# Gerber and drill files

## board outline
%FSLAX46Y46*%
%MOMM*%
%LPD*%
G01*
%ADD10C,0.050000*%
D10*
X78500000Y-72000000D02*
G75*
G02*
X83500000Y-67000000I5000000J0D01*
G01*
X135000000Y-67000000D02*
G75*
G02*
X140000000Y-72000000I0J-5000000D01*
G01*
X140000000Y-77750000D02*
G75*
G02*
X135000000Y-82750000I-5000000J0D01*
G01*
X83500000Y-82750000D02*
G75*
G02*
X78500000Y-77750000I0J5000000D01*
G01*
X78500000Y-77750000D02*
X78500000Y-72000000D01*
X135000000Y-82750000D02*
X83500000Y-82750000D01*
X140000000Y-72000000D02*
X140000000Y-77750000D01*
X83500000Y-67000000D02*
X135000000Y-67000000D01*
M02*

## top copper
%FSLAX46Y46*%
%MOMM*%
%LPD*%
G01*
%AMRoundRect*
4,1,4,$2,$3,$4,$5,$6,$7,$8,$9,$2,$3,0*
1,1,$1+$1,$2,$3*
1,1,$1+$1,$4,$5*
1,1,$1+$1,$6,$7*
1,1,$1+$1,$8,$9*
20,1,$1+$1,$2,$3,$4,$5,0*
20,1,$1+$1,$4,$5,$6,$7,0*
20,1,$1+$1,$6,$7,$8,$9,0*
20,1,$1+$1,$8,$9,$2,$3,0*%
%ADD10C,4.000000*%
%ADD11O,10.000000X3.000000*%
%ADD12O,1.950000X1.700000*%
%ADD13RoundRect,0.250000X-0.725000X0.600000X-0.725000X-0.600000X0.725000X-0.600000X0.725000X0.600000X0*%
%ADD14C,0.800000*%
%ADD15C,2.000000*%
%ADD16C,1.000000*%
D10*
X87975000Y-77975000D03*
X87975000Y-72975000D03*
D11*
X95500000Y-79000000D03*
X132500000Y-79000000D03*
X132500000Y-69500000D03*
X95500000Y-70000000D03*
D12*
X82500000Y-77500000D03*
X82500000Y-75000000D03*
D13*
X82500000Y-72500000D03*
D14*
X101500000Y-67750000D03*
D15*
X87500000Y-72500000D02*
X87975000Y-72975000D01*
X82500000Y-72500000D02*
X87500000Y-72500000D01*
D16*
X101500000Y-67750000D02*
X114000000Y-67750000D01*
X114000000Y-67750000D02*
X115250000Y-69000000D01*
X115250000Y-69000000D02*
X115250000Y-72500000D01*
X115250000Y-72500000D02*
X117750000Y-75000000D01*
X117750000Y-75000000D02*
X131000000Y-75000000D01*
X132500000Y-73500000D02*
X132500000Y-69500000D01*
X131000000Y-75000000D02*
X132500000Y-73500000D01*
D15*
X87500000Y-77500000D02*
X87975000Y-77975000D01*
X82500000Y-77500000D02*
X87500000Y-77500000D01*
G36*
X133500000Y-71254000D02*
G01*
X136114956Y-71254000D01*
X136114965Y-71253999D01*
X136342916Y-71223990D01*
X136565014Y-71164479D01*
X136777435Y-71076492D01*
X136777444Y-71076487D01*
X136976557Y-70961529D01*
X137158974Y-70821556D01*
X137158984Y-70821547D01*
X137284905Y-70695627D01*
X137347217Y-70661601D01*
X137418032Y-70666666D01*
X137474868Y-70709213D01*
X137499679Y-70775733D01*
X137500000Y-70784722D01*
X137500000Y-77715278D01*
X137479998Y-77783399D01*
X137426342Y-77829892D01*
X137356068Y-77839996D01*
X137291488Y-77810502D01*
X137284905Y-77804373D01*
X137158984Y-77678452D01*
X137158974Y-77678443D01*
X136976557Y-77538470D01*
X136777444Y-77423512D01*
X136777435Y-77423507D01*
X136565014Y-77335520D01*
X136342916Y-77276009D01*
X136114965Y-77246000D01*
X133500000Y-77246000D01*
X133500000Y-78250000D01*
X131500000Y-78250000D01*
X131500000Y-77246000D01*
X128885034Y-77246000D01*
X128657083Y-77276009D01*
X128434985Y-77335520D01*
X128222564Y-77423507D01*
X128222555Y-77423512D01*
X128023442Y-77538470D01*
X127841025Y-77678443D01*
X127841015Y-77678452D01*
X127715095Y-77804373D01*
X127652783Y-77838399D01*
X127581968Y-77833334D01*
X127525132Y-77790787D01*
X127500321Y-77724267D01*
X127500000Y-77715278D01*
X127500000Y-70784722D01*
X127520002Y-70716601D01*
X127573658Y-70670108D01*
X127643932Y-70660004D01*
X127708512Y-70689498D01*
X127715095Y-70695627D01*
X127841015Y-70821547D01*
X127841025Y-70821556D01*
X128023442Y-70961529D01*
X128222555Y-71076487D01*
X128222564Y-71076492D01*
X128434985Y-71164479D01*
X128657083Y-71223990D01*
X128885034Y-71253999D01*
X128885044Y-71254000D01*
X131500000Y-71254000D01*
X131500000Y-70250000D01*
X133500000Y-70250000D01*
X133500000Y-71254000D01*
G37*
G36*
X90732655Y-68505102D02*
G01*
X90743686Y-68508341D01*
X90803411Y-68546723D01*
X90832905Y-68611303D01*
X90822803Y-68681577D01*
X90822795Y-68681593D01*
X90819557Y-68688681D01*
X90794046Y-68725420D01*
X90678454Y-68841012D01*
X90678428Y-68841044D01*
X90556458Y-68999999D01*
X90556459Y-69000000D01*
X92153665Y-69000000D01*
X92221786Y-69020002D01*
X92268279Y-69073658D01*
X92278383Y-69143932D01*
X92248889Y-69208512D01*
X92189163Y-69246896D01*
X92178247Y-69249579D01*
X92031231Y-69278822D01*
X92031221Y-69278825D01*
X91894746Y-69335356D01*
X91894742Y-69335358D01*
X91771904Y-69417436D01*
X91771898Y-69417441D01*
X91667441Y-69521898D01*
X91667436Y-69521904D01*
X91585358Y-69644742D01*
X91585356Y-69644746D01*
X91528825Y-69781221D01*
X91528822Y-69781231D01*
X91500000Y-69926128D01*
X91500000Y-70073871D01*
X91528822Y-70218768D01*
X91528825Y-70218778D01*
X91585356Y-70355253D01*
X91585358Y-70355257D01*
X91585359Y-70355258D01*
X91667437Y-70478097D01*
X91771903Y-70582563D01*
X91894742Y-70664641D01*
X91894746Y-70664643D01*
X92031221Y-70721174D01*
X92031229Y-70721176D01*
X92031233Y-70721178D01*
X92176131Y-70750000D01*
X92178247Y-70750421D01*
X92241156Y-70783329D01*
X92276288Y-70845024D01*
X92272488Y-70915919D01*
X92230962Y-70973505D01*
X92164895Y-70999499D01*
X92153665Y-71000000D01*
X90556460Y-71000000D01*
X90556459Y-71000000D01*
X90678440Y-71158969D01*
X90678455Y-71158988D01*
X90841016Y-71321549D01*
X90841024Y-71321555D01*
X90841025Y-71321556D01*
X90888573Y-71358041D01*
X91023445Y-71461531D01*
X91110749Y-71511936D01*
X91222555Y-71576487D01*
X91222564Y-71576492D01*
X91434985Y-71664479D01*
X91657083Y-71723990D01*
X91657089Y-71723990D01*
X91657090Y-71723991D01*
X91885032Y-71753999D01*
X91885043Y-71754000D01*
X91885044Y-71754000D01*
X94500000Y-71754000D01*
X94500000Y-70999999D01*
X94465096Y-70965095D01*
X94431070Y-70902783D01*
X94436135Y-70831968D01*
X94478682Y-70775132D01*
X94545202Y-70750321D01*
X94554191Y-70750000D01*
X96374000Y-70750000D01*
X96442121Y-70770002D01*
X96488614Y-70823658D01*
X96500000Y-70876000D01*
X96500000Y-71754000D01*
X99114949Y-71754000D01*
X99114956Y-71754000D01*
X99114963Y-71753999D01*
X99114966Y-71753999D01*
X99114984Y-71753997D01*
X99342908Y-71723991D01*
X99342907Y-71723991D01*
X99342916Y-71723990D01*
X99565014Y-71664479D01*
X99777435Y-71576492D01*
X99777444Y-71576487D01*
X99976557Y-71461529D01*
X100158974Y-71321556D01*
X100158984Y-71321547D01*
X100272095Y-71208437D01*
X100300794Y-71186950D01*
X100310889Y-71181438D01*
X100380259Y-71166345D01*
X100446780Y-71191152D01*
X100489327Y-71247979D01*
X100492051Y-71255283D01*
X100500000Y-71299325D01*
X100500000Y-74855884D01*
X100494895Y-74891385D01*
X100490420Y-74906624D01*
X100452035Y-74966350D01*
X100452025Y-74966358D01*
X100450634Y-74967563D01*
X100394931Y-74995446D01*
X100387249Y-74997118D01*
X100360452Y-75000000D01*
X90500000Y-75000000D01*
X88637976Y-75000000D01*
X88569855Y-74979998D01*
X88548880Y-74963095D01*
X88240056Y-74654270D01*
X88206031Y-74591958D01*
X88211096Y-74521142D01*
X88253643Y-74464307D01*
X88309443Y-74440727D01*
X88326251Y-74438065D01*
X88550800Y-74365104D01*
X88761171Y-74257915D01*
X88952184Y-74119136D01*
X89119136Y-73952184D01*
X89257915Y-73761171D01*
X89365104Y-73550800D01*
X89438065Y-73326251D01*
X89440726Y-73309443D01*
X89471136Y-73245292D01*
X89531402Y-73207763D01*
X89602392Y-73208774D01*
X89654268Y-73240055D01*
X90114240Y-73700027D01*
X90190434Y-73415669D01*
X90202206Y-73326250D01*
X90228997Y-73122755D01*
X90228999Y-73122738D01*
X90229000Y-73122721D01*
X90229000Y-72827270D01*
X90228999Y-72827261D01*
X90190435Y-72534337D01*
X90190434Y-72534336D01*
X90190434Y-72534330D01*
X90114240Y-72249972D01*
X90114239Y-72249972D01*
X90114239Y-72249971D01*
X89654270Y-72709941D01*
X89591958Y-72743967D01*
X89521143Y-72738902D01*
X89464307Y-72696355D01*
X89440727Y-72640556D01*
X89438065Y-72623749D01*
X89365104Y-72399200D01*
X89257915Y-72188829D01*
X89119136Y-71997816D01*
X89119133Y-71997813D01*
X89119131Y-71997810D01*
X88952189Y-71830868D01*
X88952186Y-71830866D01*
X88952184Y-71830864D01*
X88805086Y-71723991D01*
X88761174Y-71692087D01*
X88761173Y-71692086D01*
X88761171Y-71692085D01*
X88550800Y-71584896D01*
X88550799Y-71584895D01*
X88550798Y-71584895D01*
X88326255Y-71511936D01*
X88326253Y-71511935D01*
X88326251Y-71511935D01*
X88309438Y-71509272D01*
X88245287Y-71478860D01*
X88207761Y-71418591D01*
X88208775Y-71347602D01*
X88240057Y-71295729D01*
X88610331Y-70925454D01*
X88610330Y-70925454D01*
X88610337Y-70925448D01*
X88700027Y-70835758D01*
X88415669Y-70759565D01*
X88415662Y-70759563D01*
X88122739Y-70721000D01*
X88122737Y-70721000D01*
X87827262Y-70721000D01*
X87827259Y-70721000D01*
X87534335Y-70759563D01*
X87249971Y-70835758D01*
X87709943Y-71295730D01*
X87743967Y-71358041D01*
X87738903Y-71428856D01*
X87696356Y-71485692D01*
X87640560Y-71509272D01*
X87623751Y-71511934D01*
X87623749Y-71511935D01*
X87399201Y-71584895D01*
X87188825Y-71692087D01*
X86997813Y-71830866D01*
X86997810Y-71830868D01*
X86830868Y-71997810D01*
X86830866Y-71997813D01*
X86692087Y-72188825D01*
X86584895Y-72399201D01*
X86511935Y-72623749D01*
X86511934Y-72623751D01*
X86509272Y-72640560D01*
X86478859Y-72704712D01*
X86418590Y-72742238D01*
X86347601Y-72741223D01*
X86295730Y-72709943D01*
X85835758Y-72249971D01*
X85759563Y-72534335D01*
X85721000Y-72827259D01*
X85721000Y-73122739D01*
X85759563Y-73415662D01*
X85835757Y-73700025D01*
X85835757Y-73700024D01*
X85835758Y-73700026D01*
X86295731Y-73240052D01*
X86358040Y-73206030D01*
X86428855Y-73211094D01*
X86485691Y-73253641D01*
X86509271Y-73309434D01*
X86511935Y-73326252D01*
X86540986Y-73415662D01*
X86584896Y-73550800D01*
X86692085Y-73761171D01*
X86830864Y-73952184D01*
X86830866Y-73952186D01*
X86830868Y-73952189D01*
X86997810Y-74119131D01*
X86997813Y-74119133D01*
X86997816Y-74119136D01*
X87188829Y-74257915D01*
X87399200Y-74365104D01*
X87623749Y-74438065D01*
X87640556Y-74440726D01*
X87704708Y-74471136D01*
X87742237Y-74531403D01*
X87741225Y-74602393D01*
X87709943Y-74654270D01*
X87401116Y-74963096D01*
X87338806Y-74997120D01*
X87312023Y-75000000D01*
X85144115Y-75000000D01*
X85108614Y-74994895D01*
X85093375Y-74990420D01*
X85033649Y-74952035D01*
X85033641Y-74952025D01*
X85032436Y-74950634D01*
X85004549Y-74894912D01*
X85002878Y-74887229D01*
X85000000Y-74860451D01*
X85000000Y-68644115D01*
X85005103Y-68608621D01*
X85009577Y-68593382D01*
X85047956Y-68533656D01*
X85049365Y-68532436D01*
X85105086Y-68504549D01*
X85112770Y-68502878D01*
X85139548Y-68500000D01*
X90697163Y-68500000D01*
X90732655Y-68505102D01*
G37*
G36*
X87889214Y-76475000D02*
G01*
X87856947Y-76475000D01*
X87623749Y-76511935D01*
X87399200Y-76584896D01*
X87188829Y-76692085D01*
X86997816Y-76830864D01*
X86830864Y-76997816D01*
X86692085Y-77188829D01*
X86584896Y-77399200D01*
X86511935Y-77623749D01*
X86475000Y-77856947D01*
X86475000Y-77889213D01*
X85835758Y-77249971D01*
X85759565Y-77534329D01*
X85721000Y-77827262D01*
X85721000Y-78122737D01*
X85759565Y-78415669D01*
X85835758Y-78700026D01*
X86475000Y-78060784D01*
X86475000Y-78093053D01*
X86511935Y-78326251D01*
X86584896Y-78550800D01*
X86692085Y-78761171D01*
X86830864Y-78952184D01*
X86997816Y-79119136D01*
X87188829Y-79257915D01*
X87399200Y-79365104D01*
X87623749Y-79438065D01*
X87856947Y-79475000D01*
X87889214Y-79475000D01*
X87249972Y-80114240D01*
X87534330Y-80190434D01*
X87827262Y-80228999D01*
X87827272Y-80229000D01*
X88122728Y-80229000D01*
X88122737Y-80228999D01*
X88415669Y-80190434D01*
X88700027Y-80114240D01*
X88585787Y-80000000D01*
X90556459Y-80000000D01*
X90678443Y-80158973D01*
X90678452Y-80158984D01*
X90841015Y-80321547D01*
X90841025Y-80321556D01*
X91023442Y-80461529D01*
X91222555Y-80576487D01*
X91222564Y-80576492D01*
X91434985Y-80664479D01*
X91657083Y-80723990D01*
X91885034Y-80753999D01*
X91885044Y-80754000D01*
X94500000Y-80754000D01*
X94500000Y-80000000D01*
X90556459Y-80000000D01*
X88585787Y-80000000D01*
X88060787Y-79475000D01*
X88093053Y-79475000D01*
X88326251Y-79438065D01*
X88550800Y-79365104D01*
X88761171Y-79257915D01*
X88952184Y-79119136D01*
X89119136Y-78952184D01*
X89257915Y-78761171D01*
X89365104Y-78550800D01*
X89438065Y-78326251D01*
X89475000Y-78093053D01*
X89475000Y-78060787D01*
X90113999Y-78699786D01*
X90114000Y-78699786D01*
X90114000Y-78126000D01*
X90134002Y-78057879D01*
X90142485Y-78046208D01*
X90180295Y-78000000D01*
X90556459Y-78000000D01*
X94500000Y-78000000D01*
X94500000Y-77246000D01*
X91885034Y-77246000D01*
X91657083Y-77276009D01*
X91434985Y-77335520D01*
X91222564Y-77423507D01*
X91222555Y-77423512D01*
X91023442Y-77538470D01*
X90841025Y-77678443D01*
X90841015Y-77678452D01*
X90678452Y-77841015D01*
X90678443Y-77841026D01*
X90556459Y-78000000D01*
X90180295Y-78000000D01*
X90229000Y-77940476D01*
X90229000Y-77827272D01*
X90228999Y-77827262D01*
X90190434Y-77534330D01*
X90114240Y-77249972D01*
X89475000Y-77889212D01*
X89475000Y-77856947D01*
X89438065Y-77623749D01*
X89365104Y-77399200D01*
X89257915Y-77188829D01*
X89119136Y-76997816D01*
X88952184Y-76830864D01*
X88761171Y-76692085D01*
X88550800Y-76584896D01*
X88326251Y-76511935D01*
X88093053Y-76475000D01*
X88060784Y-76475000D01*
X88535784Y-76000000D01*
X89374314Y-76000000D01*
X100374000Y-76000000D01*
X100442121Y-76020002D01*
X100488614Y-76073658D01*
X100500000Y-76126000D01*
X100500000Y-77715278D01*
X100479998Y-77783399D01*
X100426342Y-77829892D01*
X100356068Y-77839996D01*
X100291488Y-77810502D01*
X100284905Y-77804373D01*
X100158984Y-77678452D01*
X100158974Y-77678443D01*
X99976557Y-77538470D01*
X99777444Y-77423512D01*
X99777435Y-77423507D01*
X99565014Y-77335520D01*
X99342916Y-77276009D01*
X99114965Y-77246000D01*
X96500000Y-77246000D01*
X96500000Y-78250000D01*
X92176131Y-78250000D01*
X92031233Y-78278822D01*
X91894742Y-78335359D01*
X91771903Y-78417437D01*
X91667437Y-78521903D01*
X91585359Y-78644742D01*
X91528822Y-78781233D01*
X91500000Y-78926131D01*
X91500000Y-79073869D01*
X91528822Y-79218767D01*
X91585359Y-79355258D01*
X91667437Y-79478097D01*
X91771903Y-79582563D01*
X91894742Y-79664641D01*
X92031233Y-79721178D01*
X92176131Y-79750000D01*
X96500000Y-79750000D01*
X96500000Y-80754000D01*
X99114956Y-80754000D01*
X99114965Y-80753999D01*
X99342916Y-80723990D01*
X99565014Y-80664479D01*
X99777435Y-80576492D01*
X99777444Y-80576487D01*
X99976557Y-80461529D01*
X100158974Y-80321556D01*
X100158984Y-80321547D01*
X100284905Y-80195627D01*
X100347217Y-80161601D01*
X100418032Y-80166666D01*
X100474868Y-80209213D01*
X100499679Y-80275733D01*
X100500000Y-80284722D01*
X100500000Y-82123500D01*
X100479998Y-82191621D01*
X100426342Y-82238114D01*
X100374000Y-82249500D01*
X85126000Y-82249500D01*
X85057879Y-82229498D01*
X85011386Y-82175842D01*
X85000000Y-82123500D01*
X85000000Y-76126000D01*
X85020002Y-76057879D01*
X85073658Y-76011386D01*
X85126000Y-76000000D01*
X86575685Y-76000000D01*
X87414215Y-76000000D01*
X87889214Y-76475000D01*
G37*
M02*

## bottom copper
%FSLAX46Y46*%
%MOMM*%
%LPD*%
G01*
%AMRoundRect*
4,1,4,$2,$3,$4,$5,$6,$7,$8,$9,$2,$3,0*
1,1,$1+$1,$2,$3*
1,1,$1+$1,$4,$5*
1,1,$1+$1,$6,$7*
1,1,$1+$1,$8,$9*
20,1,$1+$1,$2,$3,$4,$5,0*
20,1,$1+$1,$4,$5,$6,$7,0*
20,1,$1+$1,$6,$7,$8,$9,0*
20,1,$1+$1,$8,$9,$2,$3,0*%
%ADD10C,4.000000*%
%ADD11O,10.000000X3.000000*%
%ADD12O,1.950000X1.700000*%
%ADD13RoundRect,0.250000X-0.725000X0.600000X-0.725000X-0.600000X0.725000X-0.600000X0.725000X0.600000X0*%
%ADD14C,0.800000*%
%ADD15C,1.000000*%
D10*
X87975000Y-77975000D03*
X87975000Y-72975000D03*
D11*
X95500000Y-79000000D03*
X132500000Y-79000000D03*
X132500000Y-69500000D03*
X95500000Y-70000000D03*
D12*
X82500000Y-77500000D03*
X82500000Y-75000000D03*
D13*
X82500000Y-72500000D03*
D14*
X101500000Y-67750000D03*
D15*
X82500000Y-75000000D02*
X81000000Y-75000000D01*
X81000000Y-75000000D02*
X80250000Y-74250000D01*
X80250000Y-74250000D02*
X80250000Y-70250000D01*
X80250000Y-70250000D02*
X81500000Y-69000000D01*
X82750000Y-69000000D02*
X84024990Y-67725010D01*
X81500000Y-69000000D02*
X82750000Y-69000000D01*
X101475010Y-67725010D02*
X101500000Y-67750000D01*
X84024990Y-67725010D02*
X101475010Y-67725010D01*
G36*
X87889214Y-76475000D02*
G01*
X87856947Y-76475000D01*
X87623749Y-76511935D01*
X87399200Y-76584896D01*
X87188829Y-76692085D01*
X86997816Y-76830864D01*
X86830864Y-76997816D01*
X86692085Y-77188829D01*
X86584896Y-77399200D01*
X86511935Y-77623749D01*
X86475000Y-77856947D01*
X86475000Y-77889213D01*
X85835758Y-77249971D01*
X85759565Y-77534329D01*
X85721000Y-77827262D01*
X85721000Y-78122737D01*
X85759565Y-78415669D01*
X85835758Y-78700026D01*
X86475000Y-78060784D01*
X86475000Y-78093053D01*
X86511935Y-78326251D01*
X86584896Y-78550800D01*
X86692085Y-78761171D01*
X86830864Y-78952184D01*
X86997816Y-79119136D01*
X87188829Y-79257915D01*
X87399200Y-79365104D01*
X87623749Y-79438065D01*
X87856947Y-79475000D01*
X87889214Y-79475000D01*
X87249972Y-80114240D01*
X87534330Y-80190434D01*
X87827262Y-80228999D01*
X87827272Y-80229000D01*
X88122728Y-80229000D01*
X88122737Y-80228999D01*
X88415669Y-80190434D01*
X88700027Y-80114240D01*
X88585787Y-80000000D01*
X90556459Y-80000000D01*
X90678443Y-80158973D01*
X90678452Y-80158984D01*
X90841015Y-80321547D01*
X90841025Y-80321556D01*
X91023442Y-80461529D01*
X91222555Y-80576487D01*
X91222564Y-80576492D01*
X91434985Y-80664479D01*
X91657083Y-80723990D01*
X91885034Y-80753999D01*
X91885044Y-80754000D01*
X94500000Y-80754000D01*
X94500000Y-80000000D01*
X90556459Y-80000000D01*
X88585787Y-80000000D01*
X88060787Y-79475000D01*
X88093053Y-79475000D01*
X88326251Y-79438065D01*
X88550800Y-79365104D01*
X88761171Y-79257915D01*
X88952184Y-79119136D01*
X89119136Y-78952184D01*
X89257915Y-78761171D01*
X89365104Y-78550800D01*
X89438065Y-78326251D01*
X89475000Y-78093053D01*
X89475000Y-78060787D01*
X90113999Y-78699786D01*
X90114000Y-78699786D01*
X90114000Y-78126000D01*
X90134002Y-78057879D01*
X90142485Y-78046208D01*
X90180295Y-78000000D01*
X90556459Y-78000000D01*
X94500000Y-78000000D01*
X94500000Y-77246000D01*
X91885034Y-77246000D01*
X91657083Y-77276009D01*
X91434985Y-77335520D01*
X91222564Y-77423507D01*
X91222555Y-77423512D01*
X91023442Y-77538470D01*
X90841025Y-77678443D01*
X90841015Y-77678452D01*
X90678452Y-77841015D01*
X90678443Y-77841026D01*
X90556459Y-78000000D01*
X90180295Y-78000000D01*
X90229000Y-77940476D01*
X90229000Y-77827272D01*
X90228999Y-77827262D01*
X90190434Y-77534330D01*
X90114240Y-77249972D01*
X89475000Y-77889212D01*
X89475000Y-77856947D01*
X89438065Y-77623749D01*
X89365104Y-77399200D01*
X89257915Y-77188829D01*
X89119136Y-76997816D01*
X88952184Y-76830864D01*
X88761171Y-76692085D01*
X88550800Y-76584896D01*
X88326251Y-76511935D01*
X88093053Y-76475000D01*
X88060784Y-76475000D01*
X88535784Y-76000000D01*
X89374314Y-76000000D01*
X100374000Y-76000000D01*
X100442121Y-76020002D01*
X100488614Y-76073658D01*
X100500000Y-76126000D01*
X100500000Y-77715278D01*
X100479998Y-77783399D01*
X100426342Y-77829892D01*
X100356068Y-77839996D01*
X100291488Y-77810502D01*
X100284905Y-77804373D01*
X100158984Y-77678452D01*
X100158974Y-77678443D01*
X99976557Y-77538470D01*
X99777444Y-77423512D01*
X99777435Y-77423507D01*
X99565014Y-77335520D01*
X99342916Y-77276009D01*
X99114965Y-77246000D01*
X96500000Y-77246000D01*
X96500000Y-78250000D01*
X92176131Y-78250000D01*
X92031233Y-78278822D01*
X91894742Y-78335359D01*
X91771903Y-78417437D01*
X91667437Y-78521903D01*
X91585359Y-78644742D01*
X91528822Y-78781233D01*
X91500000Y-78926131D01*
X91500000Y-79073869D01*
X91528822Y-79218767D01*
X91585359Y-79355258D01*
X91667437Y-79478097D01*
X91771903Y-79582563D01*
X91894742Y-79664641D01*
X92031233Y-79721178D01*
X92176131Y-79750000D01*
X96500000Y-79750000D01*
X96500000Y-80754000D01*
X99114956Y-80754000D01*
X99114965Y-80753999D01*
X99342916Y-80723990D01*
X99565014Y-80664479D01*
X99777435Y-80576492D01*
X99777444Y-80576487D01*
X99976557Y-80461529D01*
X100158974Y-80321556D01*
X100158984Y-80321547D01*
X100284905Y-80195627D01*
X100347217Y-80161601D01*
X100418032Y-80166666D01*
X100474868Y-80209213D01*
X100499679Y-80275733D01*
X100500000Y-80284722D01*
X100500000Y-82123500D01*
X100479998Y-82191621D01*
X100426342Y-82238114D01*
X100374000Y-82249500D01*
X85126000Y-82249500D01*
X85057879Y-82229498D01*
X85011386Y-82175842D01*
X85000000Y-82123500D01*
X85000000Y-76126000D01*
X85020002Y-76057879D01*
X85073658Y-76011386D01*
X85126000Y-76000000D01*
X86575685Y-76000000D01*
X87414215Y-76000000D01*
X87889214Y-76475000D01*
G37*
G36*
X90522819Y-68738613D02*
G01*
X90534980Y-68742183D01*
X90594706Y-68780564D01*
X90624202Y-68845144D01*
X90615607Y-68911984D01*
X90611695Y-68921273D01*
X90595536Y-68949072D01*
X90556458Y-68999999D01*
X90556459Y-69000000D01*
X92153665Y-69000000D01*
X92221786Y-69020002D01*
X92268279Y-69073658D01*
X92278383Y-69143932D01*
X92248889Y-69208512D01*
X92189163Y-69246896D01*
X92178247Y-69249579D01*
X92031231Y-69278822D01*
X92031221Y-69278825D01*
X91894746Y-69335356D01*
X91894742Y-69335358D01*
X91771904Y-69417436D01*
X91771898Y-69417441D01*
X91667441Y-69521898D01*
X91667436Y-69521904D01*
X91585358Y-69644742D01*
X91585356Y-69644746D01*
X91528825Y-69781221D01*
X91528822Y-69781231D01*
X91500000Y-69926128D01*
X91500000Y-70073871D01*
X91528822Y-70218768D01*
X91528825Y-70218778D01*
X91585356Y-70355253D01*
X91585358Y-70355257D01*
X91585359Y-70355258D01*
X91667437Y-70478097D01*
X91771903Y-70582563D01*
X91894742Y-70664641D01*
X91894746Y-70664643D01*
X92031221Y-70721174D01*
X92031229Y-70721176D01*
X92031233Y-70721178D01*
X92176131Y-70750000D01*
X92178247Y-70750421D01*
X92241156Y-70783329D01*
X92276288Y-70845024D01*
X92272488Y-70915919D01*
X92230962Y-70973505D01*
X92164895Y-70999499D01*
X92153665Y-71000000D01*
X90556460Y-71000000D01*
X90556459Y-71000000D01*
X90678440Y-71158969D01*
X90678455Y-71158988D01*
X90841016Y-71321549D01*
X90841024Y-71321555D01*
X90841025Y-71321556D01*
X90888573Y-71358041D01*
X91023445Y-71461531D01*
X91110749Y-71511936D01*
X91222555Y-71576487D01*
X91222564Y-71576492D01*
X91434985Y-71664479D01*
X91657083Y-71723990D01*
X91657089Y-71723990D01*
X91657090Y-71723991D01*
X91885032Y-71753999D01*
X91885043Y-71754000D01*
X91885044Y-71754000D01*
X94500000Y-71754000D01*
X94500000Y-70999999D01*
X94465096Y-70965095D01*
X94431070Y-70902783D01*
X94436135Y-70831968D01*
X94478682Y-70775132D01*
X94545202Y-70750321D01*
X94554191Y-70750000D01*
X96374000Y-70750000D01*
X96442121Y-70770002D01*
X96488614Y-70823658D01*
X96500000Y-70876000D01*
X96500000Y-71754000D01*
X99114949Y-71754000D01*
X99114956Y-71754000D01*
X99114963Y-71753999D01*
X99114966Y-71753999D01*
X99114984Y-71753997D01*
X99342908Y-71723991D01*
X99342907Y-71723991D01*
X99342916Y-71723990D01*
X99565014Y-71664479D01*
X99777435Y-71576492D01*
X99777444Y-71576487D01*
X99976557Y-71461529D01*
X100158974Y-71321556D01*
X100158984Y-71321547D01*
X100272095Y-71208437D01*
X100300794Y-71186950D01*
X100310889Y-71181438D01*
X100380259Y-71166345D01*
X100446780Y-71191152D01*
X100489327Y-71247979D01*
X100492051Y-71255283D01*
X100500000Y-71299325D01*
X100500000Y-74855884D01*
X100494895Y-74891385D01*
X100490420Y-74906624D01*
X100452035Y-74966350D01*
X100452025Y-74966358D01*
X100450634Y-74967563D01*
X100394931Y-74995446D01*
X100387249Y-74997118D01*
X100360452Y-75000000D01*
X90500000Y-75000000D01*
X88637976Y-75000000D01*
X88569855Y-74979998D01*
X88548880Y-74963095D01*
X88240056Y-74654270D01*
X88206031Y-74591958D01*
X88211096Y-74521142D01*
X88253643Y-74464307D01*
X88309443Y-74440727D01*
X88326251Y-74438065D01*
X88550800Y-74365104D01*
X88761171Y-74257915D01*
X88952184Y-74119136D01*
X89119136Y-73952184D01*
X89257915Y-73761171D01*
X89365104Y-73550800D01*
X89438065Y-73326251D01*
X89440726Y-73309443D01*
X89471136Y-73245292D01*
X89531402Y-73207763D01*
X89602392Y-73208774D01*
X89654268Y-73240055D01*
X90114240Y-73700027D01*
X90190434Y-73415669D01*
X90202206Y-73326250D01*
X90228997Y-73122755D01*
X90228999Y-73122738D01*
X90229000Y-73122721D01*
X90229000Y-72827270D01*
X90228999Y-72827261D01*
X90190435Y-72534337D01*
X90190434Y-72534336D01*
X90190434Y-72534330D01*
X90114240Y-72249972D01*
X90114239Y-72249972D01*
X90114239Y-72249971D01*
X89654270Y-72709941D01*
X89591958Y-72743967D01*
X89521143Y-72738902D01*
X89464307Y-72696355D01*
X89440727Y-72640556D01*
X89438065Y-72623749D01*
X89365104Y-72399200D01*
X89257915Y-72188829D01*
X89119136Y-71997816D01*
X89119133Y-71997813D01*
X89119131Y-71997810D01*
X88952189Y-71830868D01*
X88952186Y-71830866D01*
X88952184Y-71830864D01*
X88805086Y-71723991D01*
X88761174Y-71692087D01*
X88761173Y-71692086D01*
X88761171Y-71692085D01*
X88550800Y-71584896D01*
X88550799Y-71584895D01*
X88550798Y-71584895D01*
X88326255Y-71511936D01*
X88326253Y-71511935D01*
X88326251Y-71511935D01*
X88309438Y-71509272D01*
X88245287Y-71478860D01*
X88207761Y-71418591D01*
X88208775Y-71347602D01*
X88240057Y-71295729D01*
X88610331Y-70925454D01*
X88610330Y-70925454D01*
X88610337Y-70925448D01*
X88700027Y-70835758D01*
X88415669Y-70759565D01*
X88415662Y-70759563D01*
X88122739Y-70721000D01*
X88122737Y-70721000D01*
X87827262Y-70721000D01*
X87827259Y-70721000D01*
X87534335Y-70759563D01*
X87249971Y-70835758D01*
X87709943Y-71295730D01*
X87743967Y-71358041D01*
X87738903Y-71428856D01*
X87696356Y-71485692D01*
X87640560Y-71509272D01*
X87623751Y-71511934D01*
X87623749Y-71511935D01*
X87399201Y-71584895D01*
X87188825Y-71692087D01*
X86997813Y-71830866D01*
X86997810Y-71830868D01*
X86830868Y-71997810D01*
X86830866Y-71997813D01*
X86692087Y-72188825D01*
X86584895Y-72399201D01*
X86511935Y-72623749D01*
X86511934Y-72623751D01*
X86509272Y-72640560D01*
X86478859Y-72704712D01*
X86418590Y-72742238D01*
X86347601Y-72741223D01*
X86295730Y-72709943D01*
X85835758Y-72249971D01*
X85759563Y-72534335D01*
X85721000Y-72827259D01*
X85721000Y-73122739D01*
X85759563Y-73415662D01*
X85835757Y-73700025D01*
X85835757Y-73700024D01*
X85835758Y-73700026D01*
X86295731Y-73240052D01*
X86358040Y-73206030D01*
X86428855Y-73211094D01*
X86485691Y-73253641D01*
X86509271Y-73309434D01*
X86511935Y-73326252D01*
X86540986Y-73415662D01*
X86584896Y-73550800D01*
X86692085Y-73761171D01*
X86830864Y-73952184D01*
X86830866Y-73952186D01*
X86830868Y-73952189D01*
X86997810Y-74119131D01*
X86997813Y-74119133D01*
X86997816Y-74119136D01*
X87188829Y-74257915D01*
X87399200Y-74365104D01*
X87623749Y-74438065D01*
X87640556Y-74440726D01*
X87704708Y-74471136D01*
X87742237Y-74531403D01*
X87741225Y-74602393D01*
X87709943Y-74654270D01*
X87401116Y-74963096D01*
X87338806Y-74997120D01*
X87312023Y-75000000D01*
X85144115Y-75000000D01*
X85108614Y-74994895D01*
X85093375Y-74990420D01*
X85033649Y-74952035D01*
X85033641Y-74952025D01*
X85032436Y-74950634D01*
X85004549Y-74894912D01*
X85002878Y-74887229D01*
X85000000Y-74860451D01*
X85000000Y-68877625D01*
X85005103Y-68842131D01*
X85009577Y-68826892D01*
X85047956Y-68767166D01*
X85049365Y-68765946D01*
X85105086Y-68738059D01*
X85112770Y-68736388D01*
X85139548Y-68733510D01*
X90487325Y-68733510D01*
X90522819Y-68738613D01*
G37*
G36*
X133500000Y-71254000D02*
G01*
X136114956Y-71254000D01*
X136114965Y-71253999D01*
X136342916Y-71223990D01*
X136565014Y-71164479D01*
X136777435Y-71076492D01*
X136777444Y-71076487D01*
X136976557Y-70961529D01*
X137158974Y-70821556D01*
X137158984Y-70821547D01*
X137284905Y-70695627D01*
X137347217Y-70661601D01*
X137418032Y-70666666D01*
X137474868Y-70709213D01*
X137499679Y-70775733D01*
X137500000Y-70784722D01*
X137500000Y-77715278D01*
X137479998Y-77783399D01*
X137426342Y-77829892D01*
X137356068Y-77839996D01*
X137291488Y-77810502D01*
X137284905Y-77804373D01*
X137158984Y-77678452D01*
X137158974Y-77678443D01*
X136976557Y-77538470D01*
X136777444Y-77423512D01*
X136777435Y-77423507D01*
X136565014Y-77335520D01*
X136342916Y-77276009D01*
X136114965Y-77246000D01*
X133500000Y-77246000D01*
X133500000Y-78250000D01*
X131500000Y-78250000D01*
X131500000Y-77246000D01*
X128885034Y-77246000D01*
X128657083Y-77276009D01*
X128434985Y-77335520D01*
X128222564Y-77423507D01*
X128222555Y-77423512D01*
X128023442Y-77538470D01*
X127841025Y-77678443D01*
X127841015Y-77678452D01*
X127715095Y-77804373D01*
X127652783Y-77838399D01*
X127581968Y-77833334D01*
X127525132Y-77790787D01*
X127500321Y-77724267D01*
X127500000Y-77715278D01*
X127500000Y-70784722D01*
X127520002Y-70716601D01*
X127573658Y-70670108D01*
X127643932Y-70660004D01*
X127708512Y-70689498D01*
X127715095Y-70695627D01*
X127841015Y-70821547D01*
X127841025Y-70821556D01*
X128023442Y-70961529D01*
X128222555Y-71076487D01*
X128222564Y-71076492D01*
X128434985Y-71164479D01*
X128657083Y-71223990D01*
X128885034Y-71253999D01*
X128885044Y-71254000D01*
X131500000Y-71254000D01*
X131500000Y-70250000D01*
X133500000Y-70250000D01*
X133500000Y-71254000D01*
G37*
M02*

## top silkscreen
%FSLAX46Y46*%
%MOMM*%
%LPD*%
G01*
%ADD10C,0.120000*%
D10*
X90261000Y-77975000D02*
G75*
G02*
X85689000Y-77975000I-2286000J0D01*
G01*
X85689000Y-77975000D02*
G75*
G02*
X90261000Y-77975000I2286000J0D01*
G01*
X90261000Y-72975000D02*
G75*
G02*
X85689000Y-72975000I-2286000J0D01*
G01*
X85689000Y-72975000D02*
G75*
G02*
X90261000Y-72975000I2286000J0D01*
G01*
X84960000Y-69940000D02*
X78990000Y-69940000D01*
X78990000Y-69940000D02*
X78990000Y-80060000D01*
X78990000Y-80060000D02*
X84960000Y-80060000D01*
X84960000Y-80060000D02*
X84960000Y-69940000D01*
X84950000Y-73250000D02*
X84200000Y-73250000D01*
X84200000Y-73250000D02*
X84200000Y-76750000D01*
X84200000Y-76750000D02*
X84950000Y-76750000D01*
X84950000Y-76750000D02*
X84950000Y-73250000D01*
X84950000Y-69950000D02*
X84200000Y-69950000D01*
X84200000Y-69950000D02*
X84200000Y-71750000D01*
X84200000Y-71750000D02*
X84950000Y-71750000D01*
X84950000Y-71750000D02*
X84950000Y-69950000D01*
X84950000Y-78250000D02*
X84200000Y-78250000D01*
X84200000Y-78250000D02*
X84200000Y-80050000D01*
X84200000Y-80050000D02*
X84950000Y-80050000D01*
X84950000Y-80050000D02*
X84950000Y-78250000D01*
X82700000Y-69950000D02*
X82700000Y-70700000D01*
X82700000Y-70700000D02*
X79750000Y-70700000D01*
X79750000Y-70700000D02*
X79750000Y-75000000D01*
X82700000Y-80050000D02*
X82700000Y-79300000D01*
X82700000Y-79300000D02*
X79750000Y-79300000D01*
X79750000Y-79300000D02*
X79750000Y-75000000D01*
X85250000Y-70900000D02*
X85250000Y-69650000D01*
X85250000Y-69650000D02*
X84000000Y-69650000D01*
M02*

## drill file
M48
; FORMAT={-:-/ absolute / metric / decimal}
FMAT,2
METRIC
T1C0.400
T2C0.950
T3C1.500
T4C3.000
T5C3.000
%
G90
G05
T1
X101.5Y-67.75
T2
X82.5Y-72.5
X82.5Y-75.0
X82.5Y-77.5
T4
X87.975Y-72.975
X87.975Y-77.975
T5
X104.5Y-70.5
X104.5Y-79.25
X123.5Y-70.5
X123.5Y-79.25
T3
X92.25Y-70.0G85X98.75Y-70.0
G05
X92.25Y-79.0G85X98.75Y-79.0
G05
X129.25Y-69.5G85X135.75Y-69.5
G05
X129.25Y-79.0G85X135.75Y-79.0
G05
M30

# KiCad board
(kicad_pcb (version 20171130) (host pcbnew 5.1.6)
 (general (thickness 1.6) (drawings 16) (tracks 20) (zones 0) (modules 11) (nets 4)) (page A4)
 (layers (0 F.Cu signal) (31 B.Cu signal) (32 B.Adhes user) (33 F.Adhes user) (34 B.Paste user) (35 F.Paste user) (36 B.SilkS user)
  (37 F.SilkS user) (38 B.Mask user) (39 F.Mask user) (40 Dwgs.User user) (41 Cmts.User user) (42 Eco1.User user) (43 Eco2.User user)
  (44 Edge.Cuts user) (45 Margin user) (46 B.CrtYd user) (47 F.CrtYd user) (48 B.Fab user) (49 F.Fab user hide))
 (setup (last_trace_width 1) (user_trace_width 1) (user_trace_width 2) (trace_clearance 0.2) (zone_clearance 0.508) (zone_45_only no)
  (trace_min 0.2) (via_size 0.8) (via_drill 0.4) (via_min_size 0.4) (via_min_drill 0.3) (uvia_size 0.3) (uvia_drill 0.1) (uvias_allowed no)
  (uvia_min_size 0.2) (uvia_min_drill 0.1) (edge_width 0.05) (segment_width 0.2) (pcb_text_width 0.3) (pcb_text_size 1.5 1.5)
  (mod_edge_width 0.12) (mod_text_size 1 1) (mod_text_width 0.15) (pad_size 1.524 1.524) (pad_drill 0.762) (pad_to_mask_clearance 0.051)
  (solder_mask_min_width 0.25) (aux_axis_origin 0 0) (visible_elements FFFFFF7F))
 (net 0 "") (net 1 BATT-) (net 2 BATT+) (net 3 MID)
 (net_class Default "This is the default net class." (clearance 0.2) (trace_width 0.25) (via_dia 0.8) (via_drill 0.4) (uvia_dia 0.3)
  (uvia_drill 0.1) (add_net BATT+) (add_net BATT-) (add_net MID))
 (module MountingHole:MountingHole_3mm (layer F.Cu) (at 123.5 70.5)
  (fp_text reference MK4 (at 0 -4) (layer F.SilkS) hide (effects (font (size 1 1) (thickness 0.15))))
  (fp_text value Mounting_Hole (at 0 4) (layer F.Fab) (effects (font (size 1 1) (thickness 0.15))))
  (pad 1 np_thru_hole circle (at 0 0) (size 3 3) (drill 3) (layers *.Cu *.Mask)))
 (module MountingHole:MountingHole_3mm (layer F.Cu) (at 104.5 70.5)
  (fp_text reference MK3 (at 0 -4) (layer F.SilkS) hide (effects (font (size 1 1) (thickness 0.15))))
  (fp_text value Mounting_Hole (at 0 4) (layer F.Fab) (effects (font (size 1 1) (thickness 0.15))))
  (pad 1 np_thru_hole circle (at 0 0) (size 3 3) (drill 3) (layers *.Cu *.Mask)))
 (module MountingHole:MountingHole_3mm (layer F.Cu) (at 123.5 79.25)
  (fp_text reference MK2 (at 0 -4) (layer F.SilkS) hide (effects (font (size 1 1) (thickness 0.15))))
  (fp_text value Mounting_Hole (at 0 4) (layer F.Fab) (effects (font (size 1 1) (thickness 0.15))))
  (pad 1 np_thru_hole circle (at 0 0) (size 3 3) (drill 3) (layers *.Cu *.Mask)))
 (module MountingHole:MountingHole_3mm (layer F.Cu) (at 104.5 79.25)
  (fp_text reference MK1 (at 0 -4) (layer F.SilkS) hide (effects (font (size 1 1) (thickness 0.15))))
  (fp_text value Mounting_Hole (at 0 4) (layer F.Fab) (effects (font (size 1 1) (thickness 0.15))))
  (pad 1 np_thru_hole circle (at 0 0) (size 3 3) (drill 3) (layers *.Cu *.Mask)))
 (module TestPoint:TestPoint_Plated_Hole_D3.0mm (layer F.Cu) (at 87.975 77.975)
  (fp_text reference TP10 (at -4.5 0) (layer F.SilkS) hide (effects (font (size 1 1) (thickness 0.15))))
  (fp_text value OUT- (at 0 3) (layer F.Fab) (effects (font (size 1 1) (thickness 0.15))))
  (fp_circle (center 0 0) (end 0 -2.286) (layer F.SilkS) (width 0.12))
  (pad 1 thru_hole circle (at 0 0) (size 4 4) (drill 3) (layers *.Cu *.Mask) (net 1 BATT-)))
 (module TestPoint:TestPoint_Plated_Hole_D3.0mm (layer F.Cu) (at 87.975 72.975)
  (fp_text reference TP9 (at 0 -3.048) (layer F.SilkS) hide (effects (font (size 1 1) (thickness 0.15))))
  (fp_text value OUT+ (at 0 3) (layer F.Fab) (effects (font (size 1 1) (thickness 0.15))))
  (fp_circle (center 0 0) (end 0 -2.286) (layer F.SilkS) (width 0.12))
  (pad 1 thru_hole circle (at 0 0) (size 4 4) (drill 3) (layers *.Cu *.Mask) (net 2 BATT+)))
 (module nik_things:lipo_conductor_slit (layer F.Cu) (at 95.5 79)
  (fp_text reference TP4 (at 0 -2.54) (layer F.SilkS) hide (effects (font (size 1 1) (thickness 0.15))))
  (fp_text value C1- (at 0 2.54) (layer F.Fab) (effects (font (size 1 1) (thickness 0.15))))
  (pad 1 thru_hole oval (at 0 0) (size 10 3) (drill oval 8 1.5) (layers *.Cu *.Mask) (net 1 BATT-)))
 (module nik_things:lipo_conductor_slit (layer F.Cu) (at 132.5 79)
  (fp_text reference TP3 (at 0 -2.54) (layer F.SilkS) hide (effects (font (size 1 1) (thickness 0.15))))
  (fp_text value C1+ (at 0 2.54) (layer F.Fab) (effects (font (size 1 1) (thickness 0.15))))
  (pad 1 thru_hole oval (at 0 0) (size 10 3) (drill oval 8 1.5) (layers *.Cu *.Mask) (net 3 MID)))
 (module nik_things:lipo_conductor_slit (layer F.Cu) (at 132.5 69.5)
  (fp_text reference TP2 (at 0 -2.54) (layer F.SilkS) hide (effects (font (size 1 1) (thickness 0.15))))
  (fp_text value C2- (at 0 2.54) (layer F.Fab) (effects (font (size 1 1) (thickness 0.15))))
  (pad 1 thru_hole oval (at 0 0) (size 10 3) (drill oval 8 1.5) (layers *.Cu *.Mask) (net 3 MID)))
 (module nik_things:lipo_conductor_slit (layer F.Cu) (at 95.5 70)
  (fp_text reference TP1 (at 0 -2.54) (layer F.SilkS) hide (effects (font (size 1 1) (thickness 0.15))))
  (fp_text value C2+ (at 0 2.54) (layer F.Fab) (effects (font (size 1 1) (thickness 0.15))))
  (pad 1 thru_hole oval (at 0 0) (size 10 3) (drill oval 8 1.5) (layers *.Cu *.Mask) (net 2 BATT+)))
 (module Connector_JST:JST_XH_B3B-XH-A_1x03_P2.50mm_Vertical (layer F.Cu) (at 82.5 72.5 270)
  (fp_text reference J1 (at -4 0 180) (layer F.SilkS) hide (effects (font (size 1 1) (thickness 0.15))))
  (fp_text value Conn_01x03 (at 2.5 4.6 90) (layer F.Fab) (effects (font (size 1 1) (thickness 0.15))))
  (fp_line (start -2.56 -2.46) (end -2.56 3.51) (layer F.SilkS) (width 0.12))
  (fp_line (start -2.56 3.51) (end 7.56 3.51) (layer F.SilkS) (width 0.12))
  (fp_line (start 7.56 3.51) (end 7.56 -2.46) (layer F.SilkS) (width 0.12))
  (fp_line (start 7.56 -2.46) (end -2.56 -2.46) (layer F.SilkS) (width 0.12))
  (fp_line (start 0.75 -2.45) (end 0.75 -1.7) (layer F.SilkS) (width 0.12))
  (fp_line (start 0.75 -1.7) (end 4.25 -1.7) (layer F.SilkS) (width 0.12))
  (fp_line (start 4.25 -1.7) (end 4.25 -2.45) (layer F.SilkS) (width 0.12))
  (fp_line (start 4.25 -2.45) (end 0.75 -2.45) (layer F.SilkS) (width 0.12))
  (fp_line (start -2.55 -2.45) (end -2.55 -1.7) (layer F.SilkS) (width 0.12))
  (fp_line (start -2.55 -1.7) (end -0.75 -1.7) (layer F.SilkS) (width 0.12))
  (fp_line (start -0.75 -1.7) (end -0.75 -2.45) (layer F.SilkS) (width 0.12))
  (fp_line (start -0.75 -2.45) (end -2.55 -2.45) (layer F.SilkS) (width 0.12))
  (fp_line (start 5.75 -2.45) (end 5.75 -1.7) (layer F.SilkS) (width 0.12))
  (fp_line (start 5.75 -1.7) (end 7.55 -1.7) (layer F.SilkS) (width 0.12))
  (fp_line (start 7.55 -1.7) (end 7.55 -2.45) (layer F.SilkS) (width 0.12))
  (fp_line (start 7.55 -2.45) (end 5.75 -2.45) (layer F.SilkS) (width 0.12))
  (fp_line (start -2.55 -0.2) (end -1.8 -0.2) (layer F.SilkS) (width 0.12))
  (fp_line (start -1.8 -0.2) (end -1.8 2.75) (layer F.SilkS) (width 0.12))
  (fp_line (start -1.8 2.75) (end 2.5 2.75) (layer F.SilkS) (width 0.12))
  (fp_line (start 7.55 -0.2) (end 6.8 -0.2) (layer F.SilkS) (width 0.12))
  (fp_line (start 6.8 -0.2) (end 6.8 2.75) (layer F.SilkS) (width 0.12))
  (fp_line (start 6.8 2.75) (end 2.5 2.75) (layer F.SilkS) (width 0.12))
  (fp_line (start -1.6 -2.75) (end -2.85 -2.75) (layer F.SilkS) (width 0.12))
  (fp_line (start -2.85 -2.75) (end -2.85 -1.5) (layer F.SilkS) (width 0.12))
  (pad 3 thru_hole oval (at 5 0 270) (size 1.7 1.95) (drill 0.95) (layers *.Cu *.Mask) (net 1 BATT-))
  (pad 2 thru_hole oval (at 2.5 0 270) (size 1.7 1.95) (drill 0.95) (layers *.Cu *.Mask) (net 3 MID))
  (pad 1 thru_hole roundrect (at 0 0 270) (size 1.7 1.95) (drill 0.95) (layers *.Cu *.Mask) (roundrect_rratio 0.147059) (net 2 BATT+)))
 (gr_arc (start 83.5 72) (end 83.5 67) (angle -90) (layer Edge.Cuts) (width 0.05))
 (gr_arc (start 135 72) (end 140 72) (angle -90) (layer Edge.Cuts) (width 0.05))
 (gr_arc (start 135 77.75) (end 135 82.75) (angle -90) (layer Edge.Cuts) (width 0.05))
 (gr_arc (start 83.5 77.75) (end 78.5 77.75) (angle -90) (layer Edge.Cuts) (width 0.05))
 (gr_line (start 78.5 77.75) (end 78.5 72) (layer Edge.Cuts) (width 0.05))
 (gr_line (start 135 82.75) (end 83.5 82.75) (layer Edge.Cuts) (width 0.05))
 (gr_line (start 140 72) (end 140 77.75) (layer Edge.Cuts) (width 0.05))
 (gr_line (start 83.5 67) (end 135 67) (layer Edge.Cuts) (width 0.05))
 (segment (start 87.5 72.5) (end 87.975 72.975) (width 2) (layer F.Cu) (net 2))
 (segment (start 82.5 72.5) (end 87.5 72.5) (width 2) (layer F.Cu) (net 2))
 (via (at 101.5 67.75) (size 0.8) (drill 0.4) (layers F.Cu B.Cu) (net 3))
 (segment (start 101.5 67.75) (end 114 67.75) (width 1) (layer F.Cu) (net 3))
 (segment (start 114 67.75) (end 115.25 69) (width 1) (layer F.Cu) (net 3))
 (segment (start 115.25 69) (end 115.25 72.5) (width 1) (layer F.Cu) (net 3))
 (segment (start 115.25 72.5) (end 117.75 75) (width 1) (layer F.Cu) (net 3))
 (segment (start 117.75 75) (end 131 75) (width 1) (layer F.Cu) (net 3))
 (segment (start 132.5 73.5) (end 132.5 69.5) (width 1) (layer F.Cu) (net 3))
 (segment (start 131 75) (end 132.5 73.5) (width 1) (layer F.Cu) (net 3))
 (segment (start 82.5 75) (end 81 75) (width 1) (layer B.Cu) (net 3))
 (segment (start 81 75) (end 80.25 74.25) (width 1) (layer B.Cu) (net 3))
 (segment (start 80.25 74.25) (end 80.25 70.25) (width 1) (layer B.Cu) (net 3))
 (segment (start 80.25 70.25) (end 81.5 69) (width 1) (layer B.Cu) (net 3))
 (segment (start 82.75 69) (end 84.02499 67.72501) (width 1) (layer B.Cu) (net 3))
 (segment (start 81.5 69) (end 82.75 69) (width 1) (layer B.Cu) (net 3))
 (segment (start 101.47501 67.72501) (end 101.5 67.75) (width 1) (layer B.Cu) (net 3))
 (segment (start 84.02499 67.72501) (end 101.47501 67.72501) (width 1) (layer B.Cu) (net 3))
 (segment (start 87.5 77.5) (end 87.975 77.975) (width 2) (layer F.Cu) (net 1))
 (segment (start 82.5 77.5) (end 87.5 77.5) (width 2) (layer F.Cu) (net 1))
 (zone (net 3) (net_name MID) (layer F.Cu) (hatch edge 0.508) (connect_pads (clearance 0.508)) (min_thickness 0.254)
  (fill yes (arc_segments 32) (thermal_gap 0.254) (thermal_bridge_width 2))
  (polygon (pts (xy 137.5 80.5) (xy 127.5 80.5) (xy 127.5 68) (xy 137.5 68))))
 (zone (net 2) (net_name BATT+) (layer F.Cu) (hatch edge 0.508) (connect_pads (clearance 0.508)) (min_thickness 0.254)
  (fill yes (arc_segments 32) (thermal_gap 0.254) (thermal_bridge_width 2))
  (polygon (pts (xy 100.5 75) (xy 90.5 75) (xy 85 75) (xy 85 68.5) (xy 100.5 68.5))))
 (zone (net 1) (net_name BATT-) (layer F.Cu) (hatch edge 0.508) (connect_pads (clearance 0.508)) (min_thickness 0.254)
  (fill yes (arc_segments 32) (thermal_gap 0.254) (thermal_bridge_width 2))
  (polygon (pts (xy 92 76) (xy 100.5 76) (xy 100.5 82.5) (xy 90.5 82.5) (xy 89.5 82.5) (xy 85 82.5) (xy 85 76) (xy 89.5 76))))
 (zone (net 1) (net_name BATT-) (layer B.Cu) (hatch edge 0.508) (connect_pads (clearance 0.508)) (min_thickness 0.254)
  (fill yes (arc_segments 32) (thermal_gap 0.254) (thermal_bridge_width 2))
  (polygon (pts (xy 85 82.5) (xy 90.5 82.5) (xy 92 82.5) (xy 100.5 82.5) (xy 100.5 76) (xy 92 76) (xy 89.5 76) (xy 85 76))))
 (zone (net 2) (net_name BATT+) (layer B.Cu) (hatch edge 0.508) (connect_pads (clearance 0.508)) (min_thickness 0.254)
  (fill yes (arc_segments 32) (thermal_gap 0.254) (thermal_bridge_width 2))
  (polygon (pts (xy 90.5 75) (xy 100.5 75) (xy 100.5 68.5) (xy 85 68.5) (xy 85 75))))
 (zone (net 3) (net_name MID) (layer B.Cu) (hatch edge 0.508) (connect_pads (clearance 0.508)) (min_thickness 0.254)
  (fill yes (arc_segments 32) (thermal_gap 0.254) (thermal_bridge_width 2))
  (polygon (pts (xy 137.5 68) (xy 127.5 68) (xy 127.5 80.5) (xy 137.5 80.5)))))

